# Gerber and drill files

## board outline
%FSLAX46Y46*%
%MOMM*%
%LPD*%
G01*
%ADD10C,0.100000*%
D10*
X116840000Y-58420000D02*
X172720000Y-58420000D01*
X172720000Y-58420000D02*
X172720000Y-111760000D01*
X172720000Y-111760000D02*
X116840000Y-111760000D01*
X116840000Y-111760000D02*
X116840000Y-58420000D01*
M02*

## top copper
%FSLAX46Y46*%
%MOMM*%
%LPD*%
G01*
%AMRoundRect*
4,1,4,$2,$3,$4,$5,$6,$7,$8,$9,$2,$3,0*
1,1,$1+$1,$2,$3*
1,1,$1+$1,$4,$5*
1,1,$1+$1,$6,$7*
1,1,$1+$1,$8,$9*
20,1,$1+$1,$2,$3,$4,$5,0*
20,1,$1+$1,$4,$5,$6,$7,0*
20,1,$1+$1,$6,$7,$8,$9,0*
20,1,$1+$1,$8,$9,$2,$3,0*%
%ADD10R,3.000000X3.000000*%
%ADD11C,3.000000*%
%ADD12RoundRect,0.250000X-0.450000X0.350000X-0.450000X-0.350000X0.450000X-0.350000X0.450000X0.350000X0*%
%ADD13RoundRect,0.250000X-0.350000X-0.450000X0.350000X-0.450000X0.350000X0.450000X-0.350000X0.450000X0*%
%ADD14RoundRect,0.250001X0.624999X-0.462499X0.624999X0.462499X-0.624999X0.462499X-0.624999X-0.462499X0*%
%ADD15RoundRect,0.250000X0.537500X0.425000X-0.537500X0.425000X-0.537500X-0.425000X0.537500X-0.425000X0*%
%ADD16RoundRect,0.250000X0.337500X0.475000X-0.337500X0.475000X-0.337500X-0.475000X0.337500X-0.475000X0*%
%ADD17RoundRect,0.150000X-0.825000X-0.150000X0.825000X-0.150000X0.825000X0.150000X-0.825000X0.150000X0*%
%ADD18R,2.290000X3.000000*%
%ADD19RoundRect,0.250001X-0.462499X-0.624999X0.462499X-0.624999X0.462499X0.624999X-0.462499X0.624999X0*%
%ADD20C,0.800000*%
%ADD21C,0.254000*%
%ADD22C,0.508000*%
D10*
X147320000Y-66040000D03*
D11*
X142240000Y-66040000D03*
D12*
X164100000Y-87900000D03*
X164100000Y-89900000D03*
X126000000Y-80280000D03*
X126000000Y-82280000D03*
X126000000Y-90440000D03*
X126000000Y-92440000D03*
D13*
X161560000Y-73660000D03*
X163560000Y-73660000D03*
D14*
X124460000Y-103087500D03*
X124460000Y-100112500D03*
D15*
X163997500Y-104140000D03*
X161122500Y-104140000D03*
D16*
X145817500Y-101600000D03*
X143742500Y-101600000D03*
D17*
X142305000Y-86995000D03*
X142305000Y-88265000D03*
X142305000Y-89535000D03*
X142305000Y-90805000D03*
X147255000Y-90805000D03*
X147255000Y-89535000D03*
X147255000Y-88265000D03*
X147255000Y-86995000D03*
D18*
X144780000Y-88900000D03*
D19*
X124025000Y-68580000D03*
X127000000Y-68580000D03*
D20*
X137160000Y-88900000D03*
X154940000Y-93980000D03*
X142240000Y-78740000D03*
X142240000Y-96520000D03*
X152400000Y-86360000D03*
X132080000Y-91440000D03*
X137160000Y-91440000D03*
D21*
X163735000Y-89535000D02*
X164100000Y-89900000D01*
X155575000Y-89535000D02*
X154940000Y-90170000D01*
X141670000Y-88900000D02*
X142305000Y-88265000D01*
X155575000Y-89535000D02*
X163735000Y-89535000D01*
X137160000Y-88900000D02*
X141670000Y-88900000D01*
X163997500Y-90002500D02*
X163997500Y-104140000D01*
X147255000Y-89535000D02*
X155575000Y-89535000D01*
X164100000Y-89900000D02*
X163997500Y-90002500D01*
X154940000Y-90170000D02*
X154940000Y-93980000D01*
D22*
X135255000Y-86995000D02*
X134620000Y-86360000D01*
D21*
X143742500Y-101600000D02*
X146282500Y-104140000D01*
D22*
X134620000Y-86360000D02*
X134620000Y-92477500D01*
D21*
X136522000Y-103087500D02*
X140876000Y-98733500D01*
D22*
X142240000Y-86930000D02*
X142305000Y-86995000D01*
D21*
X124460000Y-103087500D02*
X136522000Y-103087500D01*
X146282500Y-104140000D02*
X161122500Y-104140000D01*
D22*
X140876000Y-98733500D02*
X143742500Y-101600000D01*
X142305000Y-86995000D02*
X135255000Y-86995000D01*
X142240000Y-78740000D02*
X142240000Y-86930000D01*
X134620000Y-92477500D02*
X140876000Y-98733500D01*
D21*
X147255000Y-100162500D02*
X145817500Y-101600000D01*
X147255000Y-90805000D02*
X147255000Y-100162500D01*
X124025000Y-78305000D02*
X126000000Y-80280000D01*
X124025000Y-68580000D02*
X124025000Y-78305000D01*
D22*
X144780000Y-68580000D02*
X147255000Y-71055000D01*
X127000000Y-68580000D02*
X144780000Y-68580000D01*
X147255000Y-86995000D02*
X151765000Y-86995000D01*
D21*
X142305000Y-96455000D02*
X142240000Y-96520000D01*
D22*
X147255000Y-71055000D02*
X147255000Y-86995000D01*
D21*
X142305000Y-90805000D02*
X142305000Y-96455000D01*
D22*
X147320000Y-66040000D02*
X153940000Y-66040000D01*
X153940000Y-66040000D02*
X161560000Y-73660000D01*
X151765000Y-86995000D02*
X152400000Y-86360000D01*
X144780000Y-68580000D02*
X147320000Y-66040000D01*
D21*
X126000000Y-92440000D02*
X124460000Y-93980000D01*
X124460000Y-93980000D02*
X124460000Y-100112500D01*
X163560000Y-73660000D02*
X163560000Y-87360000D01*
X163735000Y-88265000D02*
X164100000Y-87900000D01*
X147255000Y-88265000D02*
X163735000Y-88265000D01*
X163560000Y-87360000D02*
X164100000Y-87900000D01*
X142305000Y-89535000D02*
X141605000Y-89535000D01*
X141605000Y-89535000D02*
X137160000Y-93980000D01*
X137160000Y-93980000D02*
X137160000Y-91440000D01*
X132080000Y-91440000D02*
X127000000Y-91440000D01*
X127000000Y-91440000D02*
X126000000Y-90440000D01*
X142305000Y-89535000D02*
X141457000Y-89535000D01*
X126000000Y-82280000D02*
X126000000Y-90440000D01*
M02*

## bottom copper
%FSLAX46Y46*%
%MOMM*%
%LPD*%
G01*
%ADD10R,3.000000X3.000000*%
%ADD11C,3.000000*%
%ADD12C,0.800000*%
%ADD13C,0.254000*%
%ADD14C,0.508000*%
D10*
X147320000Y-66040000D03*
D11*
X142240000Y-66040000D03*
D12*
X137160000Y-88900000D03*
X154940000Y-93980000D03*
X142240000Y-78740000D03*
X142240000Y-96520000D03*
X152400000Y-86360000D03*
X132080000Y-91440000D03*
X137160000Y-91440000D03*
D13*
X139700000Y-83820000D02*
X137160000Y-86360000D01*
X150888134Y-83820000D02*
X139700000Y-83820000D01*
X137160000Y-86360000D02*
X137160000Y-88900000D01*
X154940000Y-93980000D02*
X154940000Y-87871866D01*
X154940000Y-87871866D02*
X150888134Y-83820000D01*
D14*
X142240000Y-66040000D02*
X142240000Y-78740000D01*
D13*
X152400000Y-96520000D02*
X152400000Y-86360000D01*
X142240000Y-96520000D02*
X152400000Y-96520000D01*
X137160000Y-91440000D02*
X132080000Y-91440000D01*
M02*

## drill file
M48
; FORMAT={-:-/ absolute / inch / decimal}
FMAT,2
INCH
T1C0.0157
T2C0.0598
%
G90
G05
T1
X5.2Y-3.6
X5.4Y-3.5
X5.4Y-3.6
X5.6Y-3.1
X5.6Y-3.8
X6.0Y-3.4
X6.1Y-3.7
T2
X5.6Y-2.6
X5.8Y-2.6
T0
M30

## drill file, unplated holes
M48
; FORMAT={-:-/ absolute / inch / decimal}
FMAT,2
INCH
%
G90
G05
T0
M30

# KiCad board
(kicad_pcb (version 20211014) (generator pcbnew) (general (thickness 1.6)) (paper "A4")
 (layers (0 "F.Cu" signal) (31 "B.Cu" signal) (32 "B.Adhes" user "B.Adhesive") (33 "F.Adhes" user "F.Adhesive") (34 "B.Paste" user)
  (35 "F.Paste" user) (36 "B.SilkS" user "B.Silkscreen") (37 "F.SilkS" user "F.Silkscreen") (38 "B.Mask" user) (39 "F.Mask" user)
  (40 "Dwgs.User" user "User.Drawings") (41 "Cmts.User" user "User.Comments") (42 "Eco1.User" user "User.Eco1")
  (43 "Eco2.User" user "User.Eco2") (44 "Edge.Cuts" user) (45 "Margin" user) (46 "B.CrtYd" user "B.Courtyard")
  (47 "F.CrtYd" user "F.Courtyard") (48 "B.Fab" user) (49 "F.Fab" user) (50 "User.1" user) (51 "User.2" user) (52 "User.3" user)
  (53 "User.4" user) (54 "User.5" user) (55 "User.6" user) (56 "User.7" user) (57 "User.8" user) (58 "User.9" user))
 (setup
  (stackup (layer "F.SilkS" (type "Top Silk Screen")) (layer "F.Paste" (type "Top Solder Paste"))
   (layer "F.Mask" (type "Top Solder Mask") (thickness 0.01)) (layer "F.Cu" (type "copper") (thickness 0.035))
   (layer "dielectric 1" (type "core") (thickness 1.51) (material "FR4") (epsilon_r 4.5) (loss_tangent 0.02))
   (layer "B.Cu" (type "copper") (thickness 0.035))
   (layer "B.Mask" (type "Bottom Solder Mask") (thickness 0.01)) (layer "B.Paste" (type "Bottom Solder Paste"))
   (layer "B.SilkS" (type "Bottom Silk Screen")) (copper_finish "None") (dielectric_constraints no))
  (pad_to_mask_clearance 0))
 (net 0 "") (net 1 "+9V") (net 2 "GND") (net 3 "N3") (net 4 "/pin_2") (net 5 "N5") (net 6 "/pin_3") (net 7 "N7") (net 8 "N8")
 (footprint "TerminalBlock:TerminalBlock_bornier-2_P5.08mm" (layer "F.Cu") (at 147.32 66.04 180)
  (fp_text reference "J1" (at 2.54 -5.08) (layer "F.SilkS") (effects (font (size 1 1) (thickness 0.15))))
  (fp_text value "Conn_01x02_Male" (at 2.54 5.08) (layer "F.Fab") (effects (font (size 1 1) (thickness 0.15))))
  (pad "1" thru_hole rect (at 0 0 180) (size 3 3) (drill 1.52) (layers *.Cu *.Mask) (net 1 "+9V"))
  (pad "2" thru_hole circle (at 5.08 0 180) (size 3 3) (drill 1.52) (layers *.Cu *.Mask) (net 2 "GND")))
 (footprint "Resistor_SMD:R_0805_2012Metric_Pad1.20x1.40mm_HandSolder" (layer "F.Cu") (at 164.1 88.9 -90)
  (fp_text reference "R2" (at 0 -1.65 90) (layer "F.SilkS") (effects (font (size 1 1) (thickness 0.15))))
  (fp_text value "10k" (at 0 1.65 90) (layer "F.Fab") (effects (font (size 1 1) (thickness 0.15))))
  (pad "1" smd roundrect (at -1 0 270) (size 1.2 1.4) (layers "F.Cu" "F.Paste" "F.Mask") (roundrect_rratio 0.2083333333) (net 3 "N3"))
  (pad "2" smd roundrect (at 1 0 270) (size 1.2 1.4) (layers "F.Cu" "F.Paste" "F.Mask") (roundrect_rratio 0.2083333333) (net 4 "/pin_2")))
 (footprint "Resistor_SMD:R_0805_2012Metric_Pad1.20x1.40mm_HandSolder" (layer "F.Cu") (at 126 81.28 -90)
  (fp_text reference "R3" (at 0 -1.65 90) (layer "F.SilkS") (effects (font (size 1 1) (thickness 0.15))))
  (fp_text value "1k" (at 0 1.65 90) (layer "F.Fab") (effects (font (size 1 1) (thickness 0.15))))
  (pad "1" smd roundrect (at -1 0 270) (size 1.2 1.4) (layers "F.Cu" "F.Paste" "F.Mask") (roundrect_rratio 0.2083333333) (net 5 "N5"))
  (pad "2" smd roundrect (at 1 0 270) (size 1.2 1.4) (layers "F.Cu" "F.Paste" "F.Mask") (roundrect_rratio 0.2083333333) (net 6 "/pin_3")))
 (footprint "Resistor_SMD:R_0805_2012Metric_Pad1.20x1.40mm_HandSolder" (layer "F.Cu") (at 126 91.44 -90)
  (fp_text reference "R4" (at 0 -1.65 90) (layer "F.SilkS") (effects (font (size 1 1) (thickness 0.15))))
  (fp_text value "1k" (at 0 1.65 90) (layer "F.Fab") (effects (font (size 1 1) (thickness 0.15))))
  (pad "1" smd roundrect (at -1 0 270) (size 1.2 1.4) (layers "F.Cu" "F.Paste" "F.Mask") (roundrect_rratio 0.2083333333) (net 6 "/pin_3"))
  (pad "2" smd roundrect (at 1 0 270) (size 1.2 1.4) (layers "F.Cu" "F.Paste" "F.Mask") (roundrect_rratio 0.2083333333) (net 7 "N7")))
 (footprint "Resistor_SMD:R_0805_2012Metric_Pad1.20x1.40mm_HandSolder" (layer "F.Cu") (at 162.56 73.66)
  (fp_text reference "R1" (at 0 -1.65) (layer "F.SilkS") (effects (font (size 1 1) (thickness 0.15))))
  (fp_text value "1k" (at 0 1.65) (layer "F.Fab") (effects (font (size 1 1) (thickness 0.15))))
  (pad "1" smd roundrect (at -1 0) (size 1.2 1.4) (layers "F.Cu" "F.Paste" "F.Mask") (roundrect_rratio 0.2083333333) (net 1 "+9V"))
  (pad "2" smd roundrect (at 1 0) (size 1.2 1.4) (layers "F.Cu" "F.Paste" "F.Mask") (roundrect_rratio 0.2083333333) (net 3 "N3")))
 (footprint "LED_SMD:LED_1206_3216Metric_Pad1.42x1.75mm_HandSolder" (layer "F.Cu") (at 124.46 101.6 90)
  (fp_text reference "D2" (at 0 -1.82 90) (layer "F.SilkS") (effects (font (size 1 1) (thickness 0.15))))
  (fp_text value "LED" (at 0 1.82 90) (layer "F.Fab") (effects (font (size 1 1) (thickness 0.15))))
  (pad "1" smd roundrect (at -1.4875 0 90) (size 1.425 1.75) (layers "F.Cu" "F.Paste" "F.Mask") (roundrect_rratio 0.1754392982)
   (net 2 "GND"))
  (pad "2" smd roundrect (at 1.4875 0 90) (size 1.425 1.75) (layers "F.Cu" "F.Paste" "F.Mask") (roundrect_rratio 0.1754392982) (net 7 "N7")))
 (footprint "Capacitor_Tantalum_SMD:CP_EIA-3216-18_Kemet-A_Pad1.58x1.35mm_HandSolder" (layer "F.Cu") (at 162.56 104.14 180)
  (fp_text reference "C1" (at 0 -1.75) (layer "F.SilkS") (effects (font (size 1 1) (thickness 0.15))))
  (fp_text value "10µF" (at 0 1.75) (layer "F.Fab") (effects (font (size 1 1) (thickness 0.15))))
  (pad "1" smd roundrect (at -1.4375 0 180) (size 1.575 1.35) (layers "F.Cu" "F.Paste" "F.Mask") (roundrect_rratio 0.1851851852)
   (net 4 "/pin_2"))
  (pad "2" smd roundrect (at 1.4375 0 180) (size 1.575 1.35) (layers "F.Cu" "F.Paste" "F.Mask") (roundrect_rratio 0.1851851852)
   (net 2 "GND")))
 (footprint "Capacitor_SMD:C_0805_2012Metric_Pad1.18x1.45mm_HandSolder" (layer "F.Cu") (at 144.78 101.6 180)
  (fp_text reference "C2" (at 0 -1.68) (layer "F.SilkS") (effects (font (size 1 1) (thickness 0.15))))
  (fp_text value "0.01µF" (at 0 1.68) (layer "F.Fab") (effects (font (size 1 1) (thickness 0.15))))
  (pad "1" smd roundrect (at -1.0375 0 180) (size 1.175 1.45) (layers "F.Cu" "F.Paste" "F.Mask") (roundrect_rratio 0.2127659574)
   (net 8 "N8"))
  (pad "2" smd roundrect (at 1.0375 0 180) (size 1.175 1.45) (layers "F.Cu" "F.Paste" "F.Mask") (roundrect_rratio 0.2127659574)
   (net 2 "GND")))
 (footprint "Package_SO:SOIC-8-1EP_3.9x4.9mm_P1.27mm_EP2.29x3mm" (layer "F.Cu") (at 144.78 88.9)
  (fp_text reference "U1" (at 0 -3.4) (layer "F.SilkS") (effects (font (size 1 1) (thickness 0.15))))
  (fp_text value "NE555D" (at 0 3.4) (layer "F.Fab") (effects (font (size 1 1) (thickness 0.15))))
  (pad "" smd roundrect (at 0.57 0.75) (size 0.92 1.21) (layers "F.Paste") (roundrect_rratio 0.25))
  (pad "" smd roundrect (at -0.57 -0.75) (size 0.92 1.21) (layers "F.Paste") (roundrect_rratio 0.25))
  (pad "" smd roundrect (at -0.57 0.75) (size 0.92 1.21) (layers "F.Paste") (roundrect_rratio 0.25))
  (pad "" smd roundrect (at 0.57 -0.75) (size 0.92 1.21) (layers "F.Paste") (roundrect_rratio 0.25))
  (pad "1" smd roundrect (at -2.475 -1.905) (size 1.95 0.6) (layers "F.Cu" "F.Paste" "F.Mask") (roundrect_rratio 0.25) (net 2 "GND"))
  (pad "2" smd roundrect (at -2.475 -0.635) (size 1.95 0.6) (layers "F.Cu" "F.Paste" "F.Mask") (roundrect_rratio 0.25) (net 4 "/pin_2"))
  (pad "3" smd roundrect (at -2.475 0.635) (size 1.95 0.6) (layers "F.Cu" "F.Paste" "F.Mask") (roundrect_rratio 0.25) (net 6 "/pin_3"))
  (pad "4" smd roundrect (at -2.475 1.905) (size 1.95 0.6) (layers "F.Cu" "F.Paste" "F.Mask") (roundrect_rratio 0.25) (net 1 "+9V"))
  (pad "5" smd roundrect (at 2.475 1.905) (size 1.95 0.6) (layers "F.Cu" "F.Paste" "F.Mask") (roundrect_rratio 0.25) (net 8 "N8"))
  (pad "6" smd roundrect (at 2.475 0.635) (size 1.95 0.6) (layers "F.Cu" "F.Paste" "F.Mask") (roundrect_rratio 0.25) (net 4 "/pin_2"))
  (pad "7" smd roundrect (at 2.475 -0.635) (size 1.95 0.6) (layers "F.Cu" "F.Paste" "F.Mask") (roundrect_rratio 0.25) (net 3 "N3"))
  (pad "8" smd roundrect (at 2.475 -1.905) (size 1.95 0.6) (layers "F.Cu" "F.Paste" "F.Mask") (roundrect_rratio 0.25) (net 1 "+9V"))
  (pad "9" smd rect (at 0 0) (size 2.29 3) (layers "F.Cu" "F.Mask")))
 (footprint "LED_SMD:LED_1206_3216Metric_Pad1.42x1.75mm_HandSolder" (layer "F.Cu") (at 125.5125 68.58)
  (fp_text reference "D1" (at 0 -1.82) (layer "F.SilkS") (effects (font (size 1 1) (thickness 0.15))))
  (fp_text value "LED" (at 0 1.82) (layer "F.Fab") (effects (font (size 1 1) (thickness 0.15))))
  (pad "1" smd roundrect (at -1.4875 0) (size 1.425 1.75) (layers "F.Cu" "F.Paste" "F.Mask") (roundrect_rratio 0.1754392982) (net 5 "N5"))
  (pad "2" smd roundrect (at 1.4875 0) (size 1.425 1.75) (layers "F.Cu" "F.Paste" "F.Mask") (roundrect_rratio 0.1754392982) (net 1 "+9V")))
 (gr_rect (start 116.84 58.42) (end 172.72 111.76) (layer "Edge.Cuts") (width 0.1) (fill none))
 (segment (start 163.735 89.535) (end 164.1 89.9) (width 0.254) (layer "F.Cu") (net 4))
 (segment (start 155.575 89.535) (end 154.94 90.17) (width 0.254) (layer "F.Cu") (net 4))
 (segment (start 141.67 88.9) (end 142.305 88.265) (width 0.254) (layer "F.Cu") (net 4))
 (segment (start 155.575 89.535) (end 163.735 89.535) (width 0.254) (layer "F.Cu") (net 4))
 (segment (start 137.16 88.9) (end 141.67 88.9) (width 0.254) (layer "F.Cu") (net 4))
 (segment (start 163.9975 90.0025) (end 163.9975 104.14) (width 0.254) (layer "F.Cu") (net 4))
 (segment (start 147.255 89.535) (end 155.575 89.535) (width 0.254) (layer "F.Cu") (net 4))
 (segment (start 164.1 89.9) (end 163.9975 90.0025) (width 0.254) (layer "F.Cu") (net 4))
 (segment (start 154.94 90.17) (end 154.94 93.98) (width 0.254) (layer "F.Cu") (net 4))
 (via (at 137.16 88.9) (size 0.8) (drill 0.4) (layers "F.Cu" "B.Cu") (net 4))
 (via (at 154.94 93.98) (size 0.8) (drill 0.4) (layers "F.Cu" "B.Cu") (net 4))
 (segment (start 139.7 83.82) (end 137.16 86.36) (width 0.254) (layer "B.Cu") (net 4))
 (segment (start 150.888134 83.82) (end 139.7 83.82) (width 0.254) (layer "B.Cu") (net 4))
 (segment (start 137.16 86.36) (end 137.16 88.9) (width 0.254) (layer "B.Cu") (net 4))
 (segment (start 154.94 93.98) (end 154.94 87.871866) (width 0.254) (layer "B.Cu") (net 4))
 (segment (start 154.94 87.871866) (end 150.888134 83.82) (width 0.254) (layer "B.Cu") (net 4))
 (segment (start 135.255 86.995) (end 134.62 86.36) (width 0.508) (layer "F.Cu") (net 2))
 (segment (start 143.7425 101.6) (end 146.2825 104.14) (width 0.254) (layer "F.Cu") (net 2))
 (segment (start 134.62 86.36) (end 134.62 92.4775) (width 0.508) (layer "F.Cu") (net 2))
 (segment (start 136.522 103.0875) (end 140.876 98.7335) (width 0.254) (layer "F.Cu") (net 2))
 (segment (start 142.24 86.93) (end 142.305 86.995) (width 0.508) (layer "F.Cu") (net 2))
 (segment (start 124.46 103.0875) (end 136.522 103.0875) (width 0.254) (layer "F.Cu") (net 2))
 (segment (start 146.2825 104.14) (end 161.1225 104.14) (width 0.254) (layer "F.Cu") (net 2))
 (segment (start 140.876 98.7335) (end 143.7425 101.6) (width 0.508) (layer "F.Cu") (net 2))
 (segment (start 142.305 86.995) (end 135.255 86.995) (width 0.508) (layer "F.Cu") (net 2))
 (segment (start 142.24 78.74) (end 142.24 86.93) (width 0.508) (layer "F.Cu") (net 2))
 (segment (start 134.62 92.4775) (end 140.876 98.7335) (width 0.508) (layer "F.Cu") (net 2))
 (via (at 142.24 78.74) (size 0.8) (drill 0.4) (layers "F.Cu" "B.Cu") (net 2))
 (segment (start 142.24 66.04) (end 142.24 78.74) (width 0.508) (layer "B.Cu") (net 2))
 (segment (start 147.255 100.1625) (end 145.8175 101.6) (width 0.254) (layer "F.Cu") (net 8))
 (segment (start 147.255 90.805) (end 147.255 100.1625) (width 0.254) (layer "F.Cu") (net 8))
 (segment (start 124.025 78.305) (end 126 80.28) (width 0.254) (layer "F.Cu") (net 5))
 (segment (start 124.025 68.58) (end 124.025 78.305) (width 0.254) (layer "F.Cu") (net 5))
 (segment (start 144.78 68.58) (end 147.255 71.055) (width 0.508) (layer "F.Cu") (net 1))
 (segment (start 127 68.58) (end 144.78 68.58) (width 0.508) (layer "F.Cu") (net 1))
 (segment (start 147.255 86.995) (end 151.765 86.995) (width 0.508) (layer "F.Cu") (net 1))
 (segment (start 142.305 96.455) (end 142.24 96.52) (width 0.254) (layer "F.Cu") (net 1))
 (segment (start 147.255 71.055) (end 147.255 86.995) (width 0.508) (layer "F.Cu") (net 1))
 (segment (start 142.305 90.805) (end 142.305 96.455) (width 0.254) (layer "F.Cu") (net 1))
 (segment (start 147.32 66.04) (end 153.94 66.04) (width 0.508) (layer "F.Cu") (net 1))
 (segment (start 153.94 66.04) (end 161.56 73.66) (width 0.508) (layer "F.Cu") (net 1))
 (segment (start 151.765 86.995) (end 152.4 86.36) (width 0.508) (layer "F.Cu") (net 1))
 (segment (start 144.78 68.58) (end 147.32 66.04) (width 0.508) (layer "F.Cu") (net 1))
 (via (at 142.24 96.52) (size 0.8) (drill 0.4) (layers "F.Cu" "B.Cu") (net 1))
 (via (at 152.4 86.36) (size 0.8) (drill 0.4) (layers "F.Cu" "B.Cu") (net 1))
 (segment (start 152.4 96.52) (end 152.4 86.36) (width 0.254) (layer "B.Cu") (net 1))
 (segment (start 142.24 96.52) (end 152.4 96.52) (width 0.254) (layer "B.Cu") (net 1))
 (segment (start 126 92.44) (end 124.46 93.98) (width 0.254) (layer "F.Cu") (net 7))
 (segment (start 124.46 93.98) (end 124.46 100.1125) (width 0.254) (layer "F.Cu") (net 7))
 (segment (start 163.56 73.66) (end 163.56 87.36) (width 0.254) (layer "F.Cu") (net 3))
 (segment (start 163.735 88.265) (end 164.1 87.9) (width 0.254) (layer "F.Cu") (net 3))
 (segment (start 147.255 88.265) (end 163.735 88.265) (width 0.254) (layer "F.Cu") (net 3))
 (segment (start 163.56 87.36) (end 164.1 87.9) (width 0.254) (layer "F.Cu") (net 3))
 (segment (start 142.305 89.535) (end 141.605 89.535) (width 0.254) (layer "F.Cu") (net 6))
 (segment (start 141.605 89.535) (end 137.16 93.98) (width 0.254) (layer "F.Cu") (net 6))
 (segment (start 137.16 93.98) (end 137.16 91.44) (width 0.254) (layer "F.Cu") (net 6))
 (segment (start 132.08 91.44) (end 127 91.44) (width 0.254) (layer "F.Cu") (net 6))
 (segment (start 127 91.44) (end 126 90.44) (width 0.254) (layer "F.Cu") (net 6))
 (segment (start 142.305 89.535) (end 141.457 89.535) (width 0.254) (layer "F.Cu") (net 6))
 (segment (start 126 82.28) (end 126 90.44) (width 0.254) (layer "F.Cu") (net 6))
 (via (at 132.08 91.44) (size 0.8) (drill 0.4) (layers "F.Cu" "B.Cu") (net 6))
 (via (at 137.16 91.44) (size 0.8) (drill 0.4) (layers "F.Cu" "B.Cu") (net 6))
 (segment (start 137.16 91.44) (end 132.08 91.44) (width 0.254) (layer "B.Cu") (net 6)))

